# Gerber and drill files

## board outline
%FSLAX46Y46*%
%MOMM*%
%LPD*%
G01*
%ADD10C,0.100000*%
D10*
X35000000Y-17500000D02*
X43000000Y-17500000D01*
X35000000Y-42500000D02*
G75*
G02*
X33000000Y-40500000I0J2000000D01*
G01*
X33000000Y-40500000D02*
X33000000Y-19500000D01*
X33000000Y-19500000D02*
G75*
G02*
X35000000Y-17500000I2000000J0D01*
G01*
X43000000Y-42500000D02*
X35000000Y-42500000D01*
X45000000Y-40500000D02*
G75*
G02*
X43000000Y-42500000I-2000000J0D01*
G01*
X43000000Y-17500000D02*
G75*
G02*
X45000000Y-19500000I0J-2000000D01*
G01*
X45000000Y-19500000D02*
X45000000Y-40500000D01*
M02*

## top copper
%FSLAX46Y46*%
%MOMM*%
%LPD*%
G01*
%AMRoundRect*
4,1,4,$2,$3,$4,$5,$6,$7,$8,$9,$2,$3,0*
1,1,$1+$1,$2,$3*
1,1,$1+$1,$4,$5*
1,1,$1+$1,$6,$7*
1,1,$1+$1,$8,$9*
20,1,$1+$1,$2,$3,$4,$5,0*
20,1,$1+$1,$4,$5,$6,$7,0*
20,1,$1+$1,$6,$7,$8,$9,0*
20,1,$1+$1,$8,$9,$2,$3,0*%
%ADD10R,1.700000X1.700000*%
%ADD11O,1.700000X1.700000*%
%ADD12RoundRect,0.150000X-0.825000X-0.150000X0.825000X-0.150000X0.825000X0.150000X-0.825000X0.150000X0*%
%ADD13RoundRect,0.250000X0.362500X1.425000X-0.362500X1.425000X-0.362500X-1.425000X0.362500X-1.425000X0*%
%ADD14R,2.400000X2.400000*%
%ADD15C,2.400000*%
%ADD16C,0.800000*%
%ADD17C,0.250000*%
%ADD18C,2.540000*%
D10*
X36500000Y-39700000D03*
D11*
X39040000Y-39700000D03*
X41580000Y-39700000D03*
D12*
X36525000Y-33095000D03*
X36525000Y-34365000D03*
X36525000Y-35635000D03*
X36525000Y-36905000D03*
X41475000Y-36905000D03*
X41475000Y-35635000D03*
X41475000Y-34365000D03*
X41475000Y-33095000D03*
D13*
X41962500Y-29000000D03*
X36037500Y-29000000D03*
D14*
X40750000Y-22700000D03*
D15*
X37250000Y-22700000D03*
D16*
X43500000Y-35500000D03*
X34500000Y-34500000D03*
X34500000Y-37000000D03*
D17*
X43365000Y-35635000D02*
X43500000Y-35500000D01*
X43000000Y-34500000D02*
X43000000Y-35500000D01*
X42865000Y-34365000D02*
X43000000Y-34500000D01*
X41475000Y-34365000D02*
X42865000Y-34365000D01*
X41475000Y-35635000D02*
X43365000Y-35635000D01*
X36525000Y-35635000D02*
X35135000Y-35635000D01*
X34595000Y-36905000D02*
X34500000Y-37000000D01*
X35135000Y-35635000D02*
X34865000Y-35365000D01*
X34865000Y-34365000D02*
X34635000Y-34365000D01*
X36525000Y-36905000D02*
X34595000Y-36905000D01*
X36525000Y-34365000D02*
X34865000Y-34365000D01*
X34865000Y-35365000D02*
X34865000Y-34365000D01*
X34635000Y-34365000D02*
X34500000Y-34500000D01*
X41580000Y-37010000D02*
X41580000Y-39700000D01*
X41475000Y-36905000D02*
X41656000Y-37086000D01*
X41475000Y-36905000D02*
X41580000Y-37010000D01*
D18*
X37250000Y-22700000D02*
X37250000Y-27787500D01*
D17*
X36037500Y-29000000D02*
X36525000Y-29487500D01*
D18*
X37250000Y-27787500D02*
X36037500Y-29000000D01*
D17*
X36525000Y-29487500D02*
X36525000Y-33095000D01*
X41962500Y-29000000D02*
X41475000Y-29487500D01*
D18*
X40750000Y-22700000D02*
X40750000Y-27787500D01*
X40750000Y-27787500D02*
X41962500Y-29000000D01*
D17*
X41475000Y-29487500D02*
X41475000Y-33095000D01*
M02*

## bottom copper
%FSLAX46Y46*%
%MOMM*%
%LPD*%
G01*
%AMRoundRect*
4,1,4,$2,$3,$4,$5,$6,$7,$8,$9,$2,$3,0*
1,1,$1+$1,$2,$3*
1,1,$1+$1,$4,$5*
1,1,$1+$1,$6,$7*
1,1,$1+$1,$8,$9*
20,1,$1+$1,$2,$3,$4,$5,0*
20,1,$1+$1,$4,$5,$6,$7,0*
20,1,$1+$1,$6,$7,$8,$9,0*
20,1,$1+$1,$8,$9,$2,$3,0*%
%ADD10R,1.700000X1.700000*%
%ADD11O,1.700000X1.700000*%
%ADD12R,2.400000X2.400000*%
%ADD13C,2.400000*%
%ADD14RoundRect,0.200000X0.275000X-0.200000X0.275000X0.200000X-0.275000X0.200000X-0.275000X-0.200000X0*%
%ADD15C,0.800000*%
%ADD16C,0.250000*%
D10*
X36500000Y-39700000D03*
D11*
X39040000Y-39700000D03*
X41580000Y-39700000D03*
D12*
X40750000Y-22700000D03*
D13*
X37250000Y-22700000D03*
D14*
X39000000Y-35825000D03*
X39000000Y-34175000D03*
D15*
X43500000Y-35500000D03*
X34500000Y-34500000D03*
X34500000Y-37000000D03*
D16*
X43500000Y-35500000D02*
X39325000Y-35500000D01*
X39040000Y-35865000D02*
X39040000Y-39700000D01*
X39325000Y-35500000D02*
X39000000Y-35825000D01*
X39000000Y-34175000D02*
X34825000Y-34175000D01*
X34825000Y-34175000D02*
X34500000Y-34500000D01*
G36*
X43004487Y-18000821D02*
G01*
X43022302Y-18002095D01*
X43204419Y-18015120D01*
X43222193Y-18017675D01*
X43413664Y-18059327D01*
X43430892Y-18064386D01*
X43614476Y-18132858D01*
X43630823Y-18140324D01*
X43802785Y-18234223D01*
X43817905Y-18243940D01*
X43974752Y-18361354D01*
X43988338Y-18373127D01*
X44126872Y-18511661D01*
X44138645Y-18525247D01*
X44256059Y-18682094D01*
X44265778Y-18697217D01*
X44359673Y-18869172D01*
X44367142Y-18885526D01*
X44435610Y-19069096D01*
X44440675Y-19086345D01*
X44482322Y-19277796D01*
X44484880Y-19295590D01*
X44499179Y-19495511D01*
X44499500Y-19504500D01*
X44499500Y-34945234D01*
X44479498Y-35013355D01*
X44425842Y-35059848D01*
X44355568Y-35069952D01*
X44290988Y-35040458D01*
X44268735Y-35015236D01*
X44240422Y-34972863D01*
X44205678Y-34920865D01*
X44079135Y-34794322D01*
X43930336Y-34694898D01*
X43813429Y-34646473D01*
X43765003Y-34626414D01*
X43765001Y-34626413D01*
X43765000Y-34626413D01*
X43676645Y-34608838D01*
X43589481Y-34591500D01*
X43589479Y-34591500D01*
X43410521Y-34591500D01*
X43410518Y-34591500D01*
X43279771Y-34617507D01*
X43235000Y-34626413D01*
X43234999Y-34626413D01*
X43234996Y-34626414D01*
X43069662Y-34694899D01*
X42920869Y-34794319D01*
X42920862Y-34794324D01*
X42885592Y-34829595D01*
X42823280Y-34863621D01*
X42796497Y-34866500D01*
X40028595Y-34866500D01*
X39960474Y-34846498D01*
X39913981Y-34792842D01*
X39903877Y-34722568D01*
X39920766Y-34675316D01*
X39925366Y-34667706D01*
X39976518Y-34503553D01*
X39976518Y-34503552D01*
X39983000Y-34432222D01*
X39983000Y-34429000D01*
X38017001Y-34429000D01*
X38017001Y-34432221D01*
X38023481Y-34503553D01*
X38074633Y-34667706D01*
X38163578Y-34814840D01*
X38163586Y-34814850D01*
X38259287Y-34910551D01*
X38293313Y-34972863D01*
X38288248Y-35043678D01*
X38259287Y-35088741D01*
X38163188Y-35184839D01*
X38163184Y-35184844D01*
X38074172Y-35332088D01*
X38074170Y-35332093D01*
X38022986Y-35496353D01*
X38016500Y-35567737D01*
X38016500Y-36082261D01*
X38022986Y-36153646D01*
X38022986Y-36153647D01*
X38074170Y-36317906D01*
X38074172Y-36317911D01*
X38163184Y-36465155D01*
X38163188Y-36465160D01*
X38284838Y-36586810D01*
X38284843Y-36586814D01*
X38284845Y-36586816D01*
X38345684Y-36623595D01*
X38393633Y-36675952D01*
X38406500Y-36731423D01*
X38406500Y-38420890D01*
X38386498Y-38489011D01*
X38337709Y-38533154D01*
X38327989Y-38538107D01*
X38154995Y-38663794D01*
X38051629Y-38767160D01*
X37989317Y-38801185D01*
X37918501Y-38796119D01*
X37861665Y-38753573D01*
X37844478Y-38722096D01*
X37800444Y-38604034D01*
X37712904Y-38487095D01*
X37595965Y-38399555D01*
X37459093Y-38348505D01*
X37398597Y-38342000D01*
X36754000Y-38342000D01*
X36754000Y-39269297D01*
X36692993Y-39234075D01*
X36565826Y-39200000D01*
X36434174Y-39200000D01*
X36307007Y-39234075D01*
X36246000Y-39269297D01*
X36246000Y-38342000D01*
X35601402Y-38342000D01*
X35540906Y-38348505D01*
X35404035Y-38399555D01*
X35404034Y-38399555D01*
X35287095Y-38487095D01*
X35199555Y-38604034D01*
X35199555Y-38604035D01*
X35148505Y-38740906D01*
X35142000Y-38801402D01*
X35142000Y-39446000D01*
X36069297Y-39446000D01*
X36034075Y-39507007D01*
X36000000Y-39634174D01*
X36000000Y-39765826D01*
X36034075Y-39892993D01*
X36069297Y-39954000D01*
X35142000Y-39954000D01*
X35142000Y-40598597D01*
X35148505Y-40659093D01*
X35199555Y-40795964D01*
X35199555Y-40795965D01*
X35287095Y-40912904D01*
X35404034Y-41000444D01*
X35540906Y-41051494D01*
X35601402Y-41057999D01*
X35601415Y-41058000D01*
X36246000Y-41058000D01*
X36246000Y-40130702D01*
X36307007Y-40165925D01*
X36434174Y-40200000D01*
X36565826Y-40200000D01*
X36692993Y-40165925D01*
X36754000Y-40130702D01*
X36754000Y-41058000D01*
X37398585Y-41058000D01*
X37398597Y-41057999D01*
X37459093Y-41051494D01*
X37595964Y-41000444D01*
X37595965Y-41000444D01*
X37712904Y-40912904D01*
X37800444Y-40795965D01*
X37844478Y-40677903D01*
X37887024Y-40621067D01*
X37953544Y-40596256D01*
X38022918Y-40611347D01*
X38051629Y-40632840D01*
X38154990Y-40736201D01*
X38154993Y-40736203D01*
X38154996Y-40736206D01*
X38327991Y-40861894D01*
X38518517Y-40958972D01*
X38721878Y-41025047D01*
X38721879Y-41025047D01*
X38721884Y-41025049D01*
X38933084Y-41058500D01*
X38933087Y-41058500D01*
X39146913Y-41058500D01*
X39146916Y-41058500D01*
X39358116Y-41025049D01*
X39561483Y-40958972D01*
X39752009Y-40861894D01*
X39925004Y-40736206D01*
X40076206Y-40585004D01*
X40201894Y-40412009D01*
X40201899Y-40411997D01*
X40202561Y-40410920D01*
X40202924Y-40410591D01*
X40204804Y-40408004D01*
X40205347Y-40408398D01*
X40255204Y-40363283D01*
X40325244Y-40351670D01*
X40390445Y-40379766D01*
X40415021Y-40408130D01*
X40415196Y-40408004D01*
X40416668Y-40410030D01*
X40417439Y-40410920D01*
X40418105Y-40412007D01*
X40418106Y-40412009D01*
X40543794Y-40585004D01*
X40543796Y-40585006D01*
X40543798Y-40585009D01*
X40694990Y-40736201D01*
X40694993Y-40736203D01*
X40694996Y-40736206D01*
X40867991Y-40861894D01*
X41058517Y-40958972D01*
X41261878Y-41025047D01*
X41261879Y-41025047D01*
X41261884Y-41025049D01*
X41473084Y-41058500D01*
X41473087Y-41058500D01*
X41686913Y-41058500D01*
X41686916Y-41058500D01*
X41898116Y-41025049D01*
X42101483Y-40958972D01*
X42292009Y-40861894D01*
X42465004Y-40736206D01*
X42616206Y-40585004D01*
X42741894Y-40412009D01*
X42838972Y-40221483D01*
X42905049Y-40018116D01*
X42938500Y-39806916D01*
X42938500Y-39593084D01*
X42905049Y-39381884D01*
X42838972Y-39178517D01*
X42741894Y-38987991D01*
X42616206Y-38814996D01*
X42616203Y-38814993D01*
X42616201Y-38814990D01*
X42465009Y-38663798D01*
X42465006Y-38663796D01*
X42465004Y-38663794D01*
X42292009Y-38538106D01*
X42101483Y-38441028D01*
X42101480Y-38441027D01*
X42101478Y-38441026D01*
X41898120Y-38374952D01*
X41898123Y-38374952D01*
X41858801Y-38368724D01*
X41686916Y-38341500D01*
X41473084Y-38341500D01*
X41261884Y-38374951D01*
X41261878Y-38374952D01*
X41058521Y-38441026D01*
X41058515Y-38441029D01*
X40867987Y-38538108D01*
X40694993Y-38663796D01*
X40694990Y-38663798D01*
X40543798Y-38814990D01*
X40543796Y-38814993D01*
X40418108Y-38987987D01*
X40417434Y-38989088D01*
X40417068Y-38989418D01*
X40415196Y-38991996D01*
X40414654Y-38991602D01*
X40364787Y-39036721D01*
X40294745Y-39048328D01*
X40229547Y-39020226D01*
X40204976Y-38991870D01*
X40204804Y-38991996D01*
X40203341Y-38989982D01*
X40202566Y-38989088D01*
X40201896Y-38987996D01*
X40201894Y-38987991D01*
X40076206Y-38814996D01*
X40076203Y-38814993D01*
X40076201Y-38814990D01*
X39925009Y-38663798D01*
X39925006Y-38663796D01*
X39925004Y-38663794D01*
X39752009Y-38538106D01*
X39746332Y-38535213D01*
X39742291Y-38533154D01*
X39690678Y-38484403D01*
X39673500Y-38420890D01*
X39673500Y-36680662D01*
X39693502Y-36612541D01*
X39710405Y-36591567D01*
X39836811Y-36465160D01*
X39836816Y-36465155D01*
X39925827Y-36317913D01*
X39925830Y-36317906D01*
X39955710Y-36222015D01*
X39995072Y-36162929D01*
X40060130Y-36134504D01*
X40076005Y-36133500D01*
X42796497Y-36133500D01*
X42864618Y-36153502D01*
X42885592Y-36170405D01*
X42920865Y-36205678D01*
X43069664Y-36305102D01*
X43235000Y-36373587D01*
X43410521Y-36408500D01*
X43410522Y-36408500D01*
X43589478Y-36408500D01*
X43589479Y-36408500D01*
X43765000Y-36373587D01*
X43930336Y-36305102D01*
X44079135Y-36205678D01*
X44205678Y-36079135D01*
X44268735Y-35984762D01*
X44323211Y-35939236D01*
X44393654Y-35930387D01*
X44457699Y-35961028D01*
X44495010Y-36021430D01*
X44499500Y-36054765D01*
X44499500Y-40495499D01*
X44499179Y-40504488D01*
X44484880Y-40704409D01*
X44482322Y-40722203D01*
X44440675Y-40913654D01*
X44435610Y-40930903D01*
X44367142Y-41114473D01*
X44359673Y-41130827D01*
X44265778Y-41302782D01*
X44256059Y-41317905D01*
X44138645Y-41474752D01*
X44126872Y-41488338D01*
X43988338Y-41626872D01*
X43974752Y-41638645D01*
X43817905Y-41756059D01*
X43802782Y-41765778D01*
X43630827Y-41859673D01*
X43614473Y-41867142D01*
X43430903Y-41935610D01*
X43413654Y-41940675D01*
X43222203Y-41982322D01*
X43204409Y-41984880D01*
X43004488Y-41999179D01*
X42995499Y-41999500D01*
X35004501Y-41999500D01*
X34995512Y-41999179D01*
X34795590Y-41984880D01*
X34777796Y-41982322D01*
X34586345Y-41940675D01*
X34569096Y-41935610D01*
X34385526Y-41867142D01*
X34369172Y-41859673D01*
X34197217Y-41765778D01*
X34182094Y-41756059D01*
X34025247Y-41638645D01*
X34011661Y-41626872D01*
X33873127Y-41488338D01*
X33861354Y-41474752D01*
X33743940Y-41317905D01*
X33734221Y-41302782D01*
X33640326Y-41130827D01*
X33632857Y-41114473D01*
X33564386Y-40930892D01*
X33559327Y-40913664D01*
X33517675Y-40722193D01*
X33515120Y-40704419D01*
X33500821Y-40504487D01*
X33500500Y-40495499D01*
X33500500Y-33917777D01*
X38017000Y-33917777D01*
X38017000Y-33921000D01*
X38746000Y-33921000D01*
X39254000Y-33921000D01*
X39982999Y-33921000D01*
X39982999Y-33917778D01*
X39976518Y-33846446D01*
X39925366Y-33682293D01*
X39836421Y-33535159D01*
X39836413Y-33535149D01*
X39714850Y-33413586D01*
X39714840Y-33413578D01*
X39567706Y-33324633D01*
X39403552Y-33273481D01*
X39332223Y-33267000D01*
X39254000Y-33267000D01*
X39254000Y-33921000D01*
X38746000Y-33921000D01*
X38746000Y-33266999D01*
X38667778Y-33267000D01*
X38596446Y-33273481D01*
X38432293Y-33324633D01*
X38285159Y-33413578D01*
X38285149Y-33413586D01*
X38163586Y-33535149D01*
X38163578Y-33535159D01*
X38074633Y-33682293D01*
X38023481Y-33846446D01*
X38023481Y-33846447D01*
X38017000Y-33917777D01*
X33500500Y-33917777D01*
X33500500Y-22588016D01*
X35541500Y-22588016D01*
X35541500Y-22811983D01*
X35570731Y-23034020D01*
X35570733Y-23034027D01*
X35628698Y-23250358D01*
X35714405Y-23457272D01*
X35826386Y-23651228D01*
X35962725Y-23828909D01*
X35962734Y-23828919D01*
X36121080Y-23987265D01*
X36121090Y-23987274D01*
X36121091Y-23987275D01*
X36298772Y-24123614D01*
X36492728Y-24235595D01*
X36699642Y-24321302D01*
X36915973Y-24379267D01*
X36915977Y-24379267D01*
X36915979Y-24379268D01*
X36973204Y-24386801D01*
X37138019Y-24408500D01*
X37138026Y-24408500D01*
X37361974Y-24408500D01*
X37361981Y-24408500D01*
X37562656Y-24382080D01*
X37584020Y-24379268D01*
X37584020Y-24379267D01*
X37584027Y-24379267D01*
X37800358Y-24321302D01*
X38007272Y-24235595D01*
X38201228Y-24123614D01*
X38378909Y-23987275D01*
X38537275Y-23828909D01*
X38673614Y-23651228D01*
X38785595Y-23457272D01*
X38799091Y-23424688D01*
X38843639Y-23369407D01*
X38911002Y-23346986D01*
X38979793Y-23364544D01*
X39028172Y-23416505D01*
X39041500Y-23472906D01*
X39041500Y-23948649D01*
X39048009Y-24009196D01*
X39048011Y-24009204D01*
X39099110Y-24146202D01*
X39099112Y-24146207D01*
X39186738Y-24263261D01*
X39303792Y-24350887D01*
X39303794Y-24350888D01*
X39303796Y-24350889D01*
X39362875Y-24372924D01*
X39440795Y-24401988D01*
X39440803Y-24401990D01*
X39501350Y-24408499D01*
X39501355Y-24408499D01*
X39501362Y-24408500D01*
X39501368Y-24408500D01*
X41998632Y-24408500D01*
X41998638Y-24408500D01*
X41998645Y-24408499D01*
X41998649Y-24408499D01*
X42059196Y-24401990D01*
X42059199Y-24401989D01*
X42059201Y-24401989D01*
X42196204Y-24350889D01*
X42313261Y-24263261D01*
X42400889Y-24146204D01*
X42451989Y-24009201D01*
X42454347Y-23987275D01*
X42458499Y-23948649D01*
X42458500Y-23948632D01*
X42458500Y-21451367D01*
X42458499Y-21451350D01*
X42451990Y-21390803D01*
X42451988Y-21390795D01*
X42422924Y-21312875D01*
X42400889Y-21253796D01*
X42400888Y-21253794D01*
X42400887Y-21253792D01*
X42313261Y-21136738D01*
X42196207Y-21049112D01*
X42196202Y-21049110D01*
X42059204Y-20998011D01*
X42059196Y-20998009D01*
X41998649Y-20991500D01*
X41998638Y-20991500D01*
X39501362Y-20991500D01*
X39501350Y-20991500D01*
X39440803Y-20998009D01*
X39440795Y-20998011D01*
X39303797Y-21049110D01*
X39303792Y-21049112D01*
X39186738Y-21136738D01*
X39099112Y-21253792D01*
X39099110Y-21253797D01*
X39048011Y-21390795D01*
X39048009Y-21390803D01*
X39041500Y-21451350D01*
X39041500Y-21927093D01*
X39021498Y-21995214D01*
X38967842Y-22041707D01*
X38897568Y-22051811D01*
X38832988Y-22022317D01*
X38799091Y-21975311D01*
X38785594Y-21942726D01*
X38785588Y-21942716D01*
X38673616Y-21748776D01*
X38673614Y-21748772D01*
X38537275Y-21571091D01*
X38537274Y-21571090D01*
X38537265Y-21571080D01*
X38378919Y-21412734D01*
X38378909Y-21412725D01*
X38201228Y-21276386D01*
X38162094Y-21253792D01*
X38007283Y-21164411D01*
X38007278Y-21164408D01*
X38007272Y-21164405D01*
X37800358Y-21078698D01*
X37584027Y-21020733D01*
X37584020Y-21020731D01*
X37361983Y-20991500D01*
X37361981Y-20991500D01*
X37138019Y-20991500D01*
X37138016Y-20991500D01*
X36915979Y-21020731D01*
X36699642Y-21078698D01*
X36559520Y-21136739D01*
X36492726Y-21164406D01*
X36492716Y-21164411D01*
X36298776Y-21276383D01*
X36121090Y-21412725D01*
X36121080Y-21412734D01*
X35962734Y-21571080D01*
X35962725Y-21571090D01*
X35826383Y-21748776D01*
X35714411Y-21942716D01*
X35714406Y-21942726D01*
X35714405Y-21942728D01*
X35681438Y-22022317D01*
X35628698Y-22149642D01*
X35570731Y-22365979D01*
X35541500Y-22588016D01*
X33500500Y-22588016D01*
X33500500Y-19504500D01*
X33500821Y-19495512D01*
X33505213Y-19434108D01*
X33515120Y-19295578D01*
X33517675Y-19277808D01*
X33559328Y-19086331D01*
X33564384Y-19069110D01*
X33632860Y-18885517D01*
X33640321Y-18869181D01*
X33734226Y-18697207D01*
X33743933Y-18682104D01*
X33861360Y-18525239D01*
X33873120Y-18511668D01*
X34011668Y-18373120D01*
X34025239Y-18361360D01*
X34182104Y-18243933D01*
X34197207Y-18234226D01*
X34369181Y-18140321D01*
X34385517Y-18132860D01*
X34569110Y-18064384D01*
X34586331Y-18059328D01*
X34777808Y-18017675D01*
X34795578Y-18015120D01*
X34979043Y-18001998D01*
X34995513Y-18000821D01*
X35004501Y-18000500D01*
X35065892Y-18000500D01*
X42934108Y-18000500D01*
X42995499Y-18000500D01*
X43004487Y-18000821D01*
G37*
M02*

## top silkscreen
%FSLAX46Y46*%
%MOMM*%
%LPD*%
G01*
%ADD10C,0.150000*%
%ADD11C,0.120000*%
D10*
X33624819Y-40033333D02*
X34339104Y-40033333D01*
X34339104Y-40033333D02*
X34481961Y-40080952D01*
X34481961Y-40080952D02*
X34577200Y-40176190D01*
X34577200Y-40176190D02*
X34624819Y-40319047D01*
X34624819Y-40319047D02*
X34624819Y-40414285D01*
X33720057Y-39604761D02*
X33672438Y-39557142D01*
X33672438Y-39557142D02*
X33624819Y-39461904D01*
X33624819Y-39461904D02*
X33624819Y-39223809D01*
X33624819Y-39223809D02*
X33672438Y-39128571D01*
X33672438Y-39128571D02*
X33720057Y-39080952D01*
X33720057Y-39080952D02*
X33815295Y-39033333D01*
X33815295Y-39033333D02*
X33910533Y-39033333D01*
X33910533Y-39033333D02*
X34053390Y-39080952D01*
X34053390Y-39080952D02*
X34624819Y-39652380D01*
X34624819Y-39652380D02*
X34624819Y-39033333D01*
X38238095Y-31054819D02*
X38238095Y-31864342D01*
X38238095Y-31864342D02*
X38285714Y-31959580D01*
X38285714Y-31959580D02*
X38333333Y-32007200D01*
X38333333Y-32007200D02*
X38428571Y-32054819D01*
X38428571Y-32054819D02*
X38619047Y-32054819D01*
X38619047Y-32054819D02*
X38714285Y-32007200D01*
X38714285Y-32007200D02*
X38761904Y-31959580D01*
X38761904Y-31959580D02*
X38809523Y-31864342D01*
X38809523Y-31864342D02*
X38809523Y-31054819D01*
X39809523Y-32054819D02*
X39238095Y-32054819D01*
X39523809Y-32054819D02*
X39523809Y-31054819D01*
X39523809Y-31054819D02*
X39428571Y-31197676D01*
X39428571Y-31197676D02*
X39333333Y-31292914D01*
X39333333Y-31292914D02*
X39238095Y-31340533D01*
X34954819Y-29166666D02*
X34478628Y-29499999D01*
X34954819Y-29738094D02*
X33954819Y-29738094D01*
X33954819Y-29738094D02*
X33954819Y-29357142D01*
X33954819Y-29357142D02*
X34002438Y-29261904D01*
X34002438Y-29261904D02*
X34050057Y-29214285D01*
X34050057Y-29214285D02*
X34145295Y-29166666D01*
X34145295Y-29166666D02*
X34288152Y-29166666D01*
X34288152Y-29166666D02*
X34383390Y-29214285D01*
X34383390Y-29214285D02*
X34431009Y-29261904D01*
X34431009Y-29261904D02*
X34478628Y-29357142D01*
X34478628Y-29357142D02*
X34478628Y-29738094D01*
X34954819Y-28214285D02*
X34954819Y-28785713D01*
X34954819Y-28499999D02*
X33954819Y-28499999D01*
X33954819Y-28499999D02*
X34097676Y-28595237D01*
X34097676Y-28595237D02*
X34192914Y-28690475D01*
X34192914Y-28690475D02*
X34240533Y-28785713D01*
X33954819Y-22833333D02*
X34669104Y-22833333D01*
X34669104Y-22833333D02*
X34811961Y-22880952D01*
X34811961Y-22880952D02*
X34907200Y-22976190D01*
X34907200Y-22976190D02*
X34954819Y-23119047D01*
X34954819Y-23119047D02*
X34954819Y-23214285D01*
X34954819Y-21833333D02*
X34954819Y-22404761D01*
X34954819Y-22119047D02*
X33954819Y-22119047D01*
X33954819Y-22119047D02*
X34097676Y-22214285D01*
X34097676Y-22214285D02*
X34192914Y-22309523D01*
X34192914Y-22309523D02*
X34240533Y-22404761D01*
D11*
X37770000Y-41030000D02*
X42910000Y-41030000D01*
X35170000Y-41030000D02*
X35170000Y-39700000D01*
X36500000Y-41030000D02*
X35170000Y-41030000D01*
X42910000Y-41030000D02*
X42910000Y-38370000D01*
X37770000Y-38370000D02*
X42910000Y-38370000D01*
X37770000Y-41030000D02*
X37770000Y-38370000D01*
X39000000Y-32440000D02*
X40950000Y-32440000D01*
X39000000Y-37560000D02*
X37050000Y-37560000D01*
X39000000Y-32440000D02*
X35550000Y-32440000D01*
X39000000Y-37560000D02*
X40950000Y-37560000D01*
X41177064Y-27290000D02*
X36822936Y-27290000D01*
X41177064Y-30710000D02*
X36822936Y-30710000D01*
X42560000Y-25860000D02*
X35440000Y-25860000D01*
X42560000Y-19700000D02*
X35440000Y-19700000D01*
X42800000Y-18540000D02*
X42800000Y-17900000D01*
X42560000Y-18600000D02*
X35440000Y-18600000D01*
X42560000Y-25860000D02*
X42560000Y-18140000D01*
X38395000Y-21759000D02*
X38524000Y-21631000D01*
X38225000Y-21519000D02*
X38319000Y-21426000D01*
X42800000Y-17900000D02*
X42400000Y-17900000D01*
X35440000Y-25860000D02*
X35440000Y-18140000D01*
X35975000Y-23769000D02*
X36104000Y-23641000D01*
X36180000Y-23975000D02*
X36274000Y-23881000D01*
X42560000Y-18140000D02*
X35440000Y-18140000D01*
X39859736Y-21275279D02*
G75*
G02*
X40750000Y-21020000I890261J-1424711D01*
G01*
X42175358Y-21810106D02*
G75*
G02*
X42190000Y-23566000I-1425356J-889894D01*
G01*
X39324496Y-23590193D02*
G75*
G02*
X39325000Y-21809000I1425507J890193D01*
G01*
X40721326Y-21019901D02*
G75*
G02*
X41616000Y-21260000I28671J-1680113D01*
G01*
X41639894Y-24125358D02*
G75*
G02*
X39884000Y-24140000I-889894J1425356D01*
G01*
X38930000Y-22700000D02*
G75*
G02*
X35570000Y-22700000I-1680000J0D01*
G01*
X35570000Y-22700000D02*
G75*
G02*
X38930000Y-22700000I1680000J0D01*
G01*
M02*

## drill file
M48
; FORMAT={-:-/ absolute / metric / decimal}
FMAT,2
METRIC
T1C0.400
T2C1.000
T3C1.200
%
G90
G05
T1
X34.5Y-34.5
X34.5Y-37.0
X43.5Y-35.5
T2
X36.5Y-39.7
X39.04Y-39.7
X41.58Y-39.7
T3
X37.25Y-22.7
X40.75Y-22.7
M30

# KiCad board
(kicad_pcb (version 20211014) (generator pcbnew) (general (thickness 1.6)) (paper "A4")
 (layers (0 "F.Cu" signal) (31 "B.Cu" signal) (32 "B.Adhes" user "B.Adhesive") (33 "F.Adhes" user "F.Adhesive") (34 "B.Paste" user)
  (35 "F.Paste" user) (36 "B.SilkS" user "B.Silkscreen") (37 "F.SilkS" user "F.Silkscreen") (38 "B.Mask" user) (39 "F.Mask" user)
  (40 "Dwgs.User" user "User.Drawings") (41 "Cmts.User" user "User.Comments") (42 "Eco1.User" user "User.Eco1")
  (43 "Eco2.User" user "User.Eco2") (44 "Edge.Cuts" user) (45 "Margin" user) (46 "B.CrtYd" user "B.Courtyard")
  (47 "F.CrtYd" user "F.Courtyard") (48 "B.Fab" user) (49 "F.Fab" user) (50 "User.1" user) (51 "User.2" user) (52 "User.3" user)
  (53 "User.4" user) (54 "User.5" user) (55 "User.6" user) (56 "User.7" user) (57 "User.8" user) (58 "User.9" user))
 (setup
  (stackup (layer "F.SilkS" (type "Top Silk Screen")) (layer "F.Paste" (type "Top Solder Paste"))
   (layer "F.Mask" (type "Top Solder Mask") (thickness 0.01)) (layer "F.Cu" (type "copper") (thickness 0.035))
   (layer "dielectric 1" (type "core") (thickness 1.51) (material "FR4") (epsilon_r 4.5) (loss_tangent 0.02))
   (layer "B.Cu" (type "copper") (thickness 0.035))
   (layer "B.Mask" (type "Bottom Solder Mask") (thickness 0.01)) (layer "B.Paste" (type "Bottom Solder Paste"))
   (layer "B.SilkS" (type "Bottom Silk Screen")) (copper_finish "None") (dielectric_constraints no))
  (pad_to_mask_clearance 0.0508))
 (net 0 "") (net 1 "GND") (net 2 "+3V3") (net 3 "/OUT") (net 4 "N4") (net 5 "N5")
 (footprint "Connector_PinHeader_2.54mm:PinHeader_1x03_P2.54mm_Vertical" (layer "F.Cu") (at 36.5 39.7 90)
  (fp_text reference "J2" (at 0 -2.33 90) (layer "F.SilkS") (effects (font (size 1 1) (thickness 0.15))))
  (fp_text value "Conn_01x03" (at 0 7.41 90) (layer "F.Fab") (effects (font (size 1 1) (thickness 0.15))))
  (fp_line (start -1.33 1.27) (end -1.33 6.41) (layer "F.SilkS") (width 0.12))
  (fp_line (start -1.33 -1.33) (end 0 -1.33) (layer "F.SilkS") (width 0.12))
  (fp_line (start -1.33 0) (end -1.33 -1.33) (layer "F.SilkS") (width 0.12))
  (fp_line (start -1.33 6.41) (end 1.33 6.41) (layer "F.SilkS") (width 0.12))
  (fp_line (start 1.33 1.27) (end 1.33 6.41) (layer "F.SilkS") (width 0.12))
  (fp_line (start -1.33 1.27) (end 1.33 1.27) (layer "F.SilkS") (width 0.12))
  (pad "1" thru_hole rect (at 0 0 90) (size 1.7 1.7) (drill 1) (layers *.Cu *.Mask) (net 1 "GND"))
  (pad "2" thru_hole oval (at 0 2.54 90) (size 1.7 1.7) (drill 1) (layers *.Cu *.Mask) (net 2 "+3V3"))
  (pad "3" thru_hole oval (at 0 5.08 90) (size 1.7 1.7) (drill 1) (layers *.Cu *.Mask) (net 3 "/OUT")))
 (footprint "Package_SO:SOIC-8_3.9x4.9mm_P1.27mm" (layer "F.Cu") (at 39 35)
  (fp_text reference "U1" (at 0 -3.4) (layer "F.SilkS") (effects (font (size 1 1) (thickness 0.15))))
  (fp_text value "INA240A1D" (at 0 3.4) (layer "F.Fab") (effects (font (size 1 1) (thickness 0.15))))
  (fp_line (start 0 -2.56) (end 1.95 -2.56) (layer "F.SilkS") (width 0.12))
  (fp_line (start 0 2.56) (end -1.95 2.56) (layer "F.SilkS") (width 0.12))
  (fp_line (start 0 -2.56) (end -3.45 -2.56) (layer "F.SilkS") (width 0.12))
  (fp_line (start 0 2.56) (end 1.95 2.56) (layer "F.SilkS") (width 0.12))
  (pad "1" smd roundrect (at -2.475 -1.905) (size 1.95 0.6) (layers "F.Cu" "F.Paste" "F.Mask") (roundrect_rratio 0.25) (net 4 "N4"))
  (pad "2" smd roundrect (at -2.475 -0.635) (size 1.95 0.6) (layers "F.Cu" "F.Paste" "F.Mask") (roundrect_rratio 0.25) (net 1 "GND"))
  (pad "3" smd roundrect (at -2.475 0.635) (size 1.95 0.6) (layers "F.Cu" "F.Paste" "F.Mask") (roundrect_rratio 0.25) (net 1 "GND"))
  (pad "4" smd roundrect (at -2.475 1.905) (size 1.95 0.6) (layers "F.Cu" "F.Paste" "F.Mask") (roundrect_rratio 0.25) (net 1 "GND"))
  (pad "5" smd roundrect (at 2.475 1.905) (size 1.95 0.6) (layers "F.Cu" "F.Paste" "F.Mask") (roundrect_rratio 0.25) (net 3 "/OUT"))
  (pad "6" smd roundrect (at 2.475 0.635) (size 1.95 0.6) (layers "F.Cu" "F.Paste" "F.Mask") (roundrect_rratio 0.25) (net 2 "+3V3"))
  (pad "7" smd roundrect (at 2.475 -0.635) (size 1.95 0.6) (layers "F.Cu" "F.Paste" "F.Mask") (roundrect_rratio 0.25) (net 2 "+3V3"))
  (pad "8" smd roundrect (at 2.475 -1.905) (size 1.95 0.6) (layers "F.Cu" "F.Paste" "F.Mask") (roundrect_rratio 0.25) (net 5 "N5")))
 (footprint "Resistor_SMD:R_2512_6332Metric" (layer "F.Cu") (at 39 29 180)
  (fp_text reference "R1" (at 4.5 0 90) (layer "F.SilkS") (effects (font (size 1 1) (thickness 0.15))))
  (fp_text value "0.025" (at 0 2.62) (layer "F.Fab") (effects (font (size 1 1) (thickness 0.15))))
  (fp_line (start -2.177064 1.71) (end 2.177064 1.71) (layer "F.SilkS") (width 0.12))
  (fp_line (start -2.177064 -1.71) (end 2.177064 -1.71) (layer "F.SilkS") (width 0.12))
  (pad "1" smd roundrect (at -2.9625 0 180) (size 1.225 3.35) (layers "F.Cu" "F.Paste" "F.Mask") (roundrect_rratio 0.2040816327)
   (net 5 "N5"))
  (pad "2" smd roundrect (at 2.9625 0 180) (size 1.225 3.35) (layers "F.Cu" "F.Paste" "F.Mask") (roundrect_rratio 0.2040816327) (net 4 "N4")))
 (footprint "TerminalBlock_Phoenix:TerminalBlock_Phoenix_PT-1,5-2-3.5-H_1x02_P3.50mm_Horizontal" (layer "F.Cu") (at 40.75 22.7 180)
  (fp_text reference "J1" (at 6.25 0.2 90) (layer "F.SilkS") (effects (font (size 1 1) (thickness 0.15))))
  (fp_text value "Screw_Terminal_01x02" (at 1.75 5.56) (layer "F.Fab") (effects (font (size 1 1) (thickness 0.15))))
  (fp_line (start -1.81 -3.16) (end 5.31 -3.16) (layer "F.SilkS") (width 0.12))
  (fp_line (start -1.81 3) (end 5.31 3) (layer "F.SilkS") (width 0.12))
  (fp_line (start -2.05 4.16) (end -2.05 4.8) (layer "F.SilkS") (width 0.12))
  (fp_line (start -1.81 4.1) (end 5.31 4.1) (layer "F.SilkS") (width 0.12))
  (fp_line (start -1.81 -3.16) (end -1.81 4.56) (layer "F.SilkS") (width 0.12))
  (fp_line (start 2.355 0.941) (end 2.226 1.069) (layer "F.SilkS") (width 0.12))
  (fp_line (start 2.525 1.181) (end 2.431 1.274) (layer "F.SilkS") (width 0.12))
  (fp_line (start -2.05 4.8) (end -1.65 4.8) (layer "F.SilkS") (width 0.12))
  (fp_line (start 5.31 -3.16) (end 5.31 4.56) (layer "F.SilkS") (width 0.12))
  (fp_line (start 4.775 -1.069) (end 4.646 -0.941) (layer "F.SilkS") (width 0.12))
  (fp_line (start 4.57 -1.275) (end 4.476 -1.181) (layer "F.SilkS") (width 0.12))
  (fp_line (start -1.81 4.56) (end 5.31 4.56) (layer "F.SilkS") (width 0.12))
  (fp_arc (start 0.890264 1.424721) (mid 0.463071 1.61492) (end 0 1.68) (layer "F.SilkS") (width 0.12))
  (fp_arc (start -1.425358 0.889894) (mid -1.680286 0.014012) (end -1.44 -0.866) (layer "F.SilkS") (width 0.12))
  (fp_arc (start 1.425504 -0.890193) (mid 1.680626 0.000476) (end 1.425 0.891) (layer "F.SilkS") (width 0.12))
  (fp_arc (start 0.028674 1.680099) (mid -0.435535 1.622918) (end -0.866 1.44) (layer "F.SilkS") (width 0.12))
  (fp_arc (start -0.889894 -1.425358) (mid -0.014012 -1.680286) (end 0.866 -1.44) (layer "F.SilkS") (width 0.12))
  (fp_circle (center 3.5 0) (end 5.18 0) (layer "F.SilkS") (width 0.12) (fill none))
  (pad "1" thru_hole rect (at 0 0 180) (size 2.4 2.4) (drill 1.2) (layers *.Cu *.Mask) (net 5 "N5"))
  (pad "2" thru_hole circle (at 3.5 0 180) (size 2.4 2.4) (drill 1.2) (layers *.Cu *.Mask) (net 4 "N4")))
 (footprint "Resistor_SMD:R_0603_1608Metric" (layer "B.Cu") (at 39 35 90)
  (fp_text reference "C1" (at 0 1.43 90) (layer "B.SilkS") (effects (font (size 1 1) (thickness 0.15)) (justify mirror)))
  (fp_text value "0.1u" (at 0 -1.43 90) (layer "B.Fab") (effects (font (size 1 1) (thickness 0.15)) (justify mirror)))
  (pad "1" smd roundrect (at -0.825 0 90) (size 0.8 0.95) (layers "B.Cu" "B.Paste" "B.Mask") (roundrect_rratio 0.25) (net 2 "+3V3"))
  (pad "2" smd roundrect (at 0.825 0 90) (size 0.8 0.95) (layers "B.Cu" "B.Paste" "B.Mask") (roundrect_rratio 0.25) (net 1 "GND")))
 (gr_line (start 35 17.5) (end 43 17.5) (layer "Edge.Cuts") (width 0.1))
 (gr_arc (start 35 42.5) (mid 33.585786 41.914214) (end 33 40.5) (layer "Edge.Cuts") (width 0.1))
 (gr_line (start 33 40.5) (end 33 19.5) (layer "Edge.Cuts") (width 0.1))
 (gr_arc (start 33 19.5) (mid 33.585786 18.085786) (end 35 17.5) (layer "Edge.Cuts") (width 0.1))
 (gr_line (start 43 42.5) (end 35 42.5) (layer "Edge.Cuts") (width 0.1))
 (gr_arc (start 45 40.5) (mid 44.414214 41.914214) (end 43 42.5) (layer "Edge.Cuts") (width 0.1))
 (gr_arc (start 43 17.5) (mid 44.414214 18.085786) (end 45 19.5) (layer "Edge.Cuts") (width 0.1))
 (gr_line (start 45 19.5) (end 45 40.5) (layer "Edge.Cuts") (width 0.1))
 (segment (start 43.365 35.635) (end 43.5 35.5) (width 0.25) (layer "F.Cu") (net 2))
 (segment (start 43 34.5) (end 43 35.5) (width 0.25) (layer "F.Cu") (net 2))
 (segment (start 42.865 34.365) (end 43 34.5) (width 0.25) (layer "F.Cu") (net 2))
 (segment (start 41.475 34.365) (end 42.865 34.365) (width 0.25) (layer "F.Cu") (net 2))
 (segment (start 41.475 35.635) (end 43.365 35.635) (width 0.25) (layer "F.Cu") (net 2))
 (via (at 43.5 35.5) (size 0.8) (drill 0.4) (layers "F.Cu" "B.Cu") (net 2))
 (segment (start 43.5 35.5) (end 39.325 35.5) (width 0.25) (layer "B.Cu") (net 2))
 (segment (start 39.04 35.865) (end 39.04 39.7) (width 0.25) (layer "B.Cu") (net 2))
 (segment (start 39.325 35.5) (end 39 35.825) (width 0.25) (layer "B.Cu") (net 2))
 (segment (start 36.525 35.635) (end 35.135 35.635) (width 0.25) (layer "F.Cu") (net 1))
 (segment (start 34.595 36.905) (end 34.5 37) (width 0.25) (layer "F.Cu") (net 1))
 (segment (start 35.135 35.635) (end 34.865 35.365) (width 0.25) (layer "F.Cu") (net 1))
 (segment (start 34.865 34.365) (end 34.635 34.365) (width 0.25) (layer "F.Cu") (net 1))
 (segment (start 36.525 36.905) (end 34.595 36.905) (width 0.25) (layer "F.Cu") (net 1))
 (segment (start 36.525 34.365) (end 34.865 34.365) (width 0.25) (layer "F.Cu") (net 1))
 (segment (start 34.865 35.365) (end 34.865 34.365) (width 0.25) (layer "F.Cu") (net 1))
 (segment (start 34.635 34.365) (end 34.5 34.5) (width 0.25) (layer "F.Cu") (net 1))
 (via (at 34.5 34.5) (size 0.8) (drill 0.4) (layers "F.Cu" "B.Cu") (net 1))
 (via (at 34.5 37) (size 0.8) (drill 0.4) (layers "F.Cu" "B.Cu") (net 1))
 (segment (start 39 34.175) (end 34.825 34.175) (width 0.25) (layer "B.Cu") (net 1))
 (segment (start 34.825 34.175) (end 34.5 34.5) (width 0.25) (layer "B.Cu") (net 1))
 (segment (start 41.58 37.01) (end 41.58 39.7) (width 0.25) (layer "F.Cu") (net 3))
 (segment (start 41.475 36.905) (end 41.656 37.086) (width 0.25) (layer "F.Cu") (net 3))
 (segment (start 41.475 36.905) (end 41.58 37.01) (width 0.25) (layer "F.Cu") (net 3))
 (segment (start 37.25 22.7) (end 37.25 27.7875) (width 2.54) (layer "F.Cu") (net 4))
 (segment (start 36.0375 29) (end 36.525 29.4875) (width 0.25) (layer "F.Cu") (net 4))
 (segment (start 37.25 27.7875) (end 36.0375 29) (width 2.54) (layer "F.Cu") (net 4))
 (segment (start 36.525 29.4875) (end 36.525 33.095) (width 0.25) (layer "F.Cu") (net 4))
 (segment (start 41.9625 29) (end 41.475 29.4875) (width 0.25) (layer "F.Cu") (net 5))
 (segment (start 40.75 22.7) (end 40.75 27.7875) (width 2.54) (layer "F.Cu") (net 5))
 (segment (start 40.75 27.7875) (end 41.9625 29) (width 2.54) (layer "F.Cu") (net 5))
 (segment (start 41.475 29.4875) (end 41.475 33.095) (width 0.25) (layer "F.Cu") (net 5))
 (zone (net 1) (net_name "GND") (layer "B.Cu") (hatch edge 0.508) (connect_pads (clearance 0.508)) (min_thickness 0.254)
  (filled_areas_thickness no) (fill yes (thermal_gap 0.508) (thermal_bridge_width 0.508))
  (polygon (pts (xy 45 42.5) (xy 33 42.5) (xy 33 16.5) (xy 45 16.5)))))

